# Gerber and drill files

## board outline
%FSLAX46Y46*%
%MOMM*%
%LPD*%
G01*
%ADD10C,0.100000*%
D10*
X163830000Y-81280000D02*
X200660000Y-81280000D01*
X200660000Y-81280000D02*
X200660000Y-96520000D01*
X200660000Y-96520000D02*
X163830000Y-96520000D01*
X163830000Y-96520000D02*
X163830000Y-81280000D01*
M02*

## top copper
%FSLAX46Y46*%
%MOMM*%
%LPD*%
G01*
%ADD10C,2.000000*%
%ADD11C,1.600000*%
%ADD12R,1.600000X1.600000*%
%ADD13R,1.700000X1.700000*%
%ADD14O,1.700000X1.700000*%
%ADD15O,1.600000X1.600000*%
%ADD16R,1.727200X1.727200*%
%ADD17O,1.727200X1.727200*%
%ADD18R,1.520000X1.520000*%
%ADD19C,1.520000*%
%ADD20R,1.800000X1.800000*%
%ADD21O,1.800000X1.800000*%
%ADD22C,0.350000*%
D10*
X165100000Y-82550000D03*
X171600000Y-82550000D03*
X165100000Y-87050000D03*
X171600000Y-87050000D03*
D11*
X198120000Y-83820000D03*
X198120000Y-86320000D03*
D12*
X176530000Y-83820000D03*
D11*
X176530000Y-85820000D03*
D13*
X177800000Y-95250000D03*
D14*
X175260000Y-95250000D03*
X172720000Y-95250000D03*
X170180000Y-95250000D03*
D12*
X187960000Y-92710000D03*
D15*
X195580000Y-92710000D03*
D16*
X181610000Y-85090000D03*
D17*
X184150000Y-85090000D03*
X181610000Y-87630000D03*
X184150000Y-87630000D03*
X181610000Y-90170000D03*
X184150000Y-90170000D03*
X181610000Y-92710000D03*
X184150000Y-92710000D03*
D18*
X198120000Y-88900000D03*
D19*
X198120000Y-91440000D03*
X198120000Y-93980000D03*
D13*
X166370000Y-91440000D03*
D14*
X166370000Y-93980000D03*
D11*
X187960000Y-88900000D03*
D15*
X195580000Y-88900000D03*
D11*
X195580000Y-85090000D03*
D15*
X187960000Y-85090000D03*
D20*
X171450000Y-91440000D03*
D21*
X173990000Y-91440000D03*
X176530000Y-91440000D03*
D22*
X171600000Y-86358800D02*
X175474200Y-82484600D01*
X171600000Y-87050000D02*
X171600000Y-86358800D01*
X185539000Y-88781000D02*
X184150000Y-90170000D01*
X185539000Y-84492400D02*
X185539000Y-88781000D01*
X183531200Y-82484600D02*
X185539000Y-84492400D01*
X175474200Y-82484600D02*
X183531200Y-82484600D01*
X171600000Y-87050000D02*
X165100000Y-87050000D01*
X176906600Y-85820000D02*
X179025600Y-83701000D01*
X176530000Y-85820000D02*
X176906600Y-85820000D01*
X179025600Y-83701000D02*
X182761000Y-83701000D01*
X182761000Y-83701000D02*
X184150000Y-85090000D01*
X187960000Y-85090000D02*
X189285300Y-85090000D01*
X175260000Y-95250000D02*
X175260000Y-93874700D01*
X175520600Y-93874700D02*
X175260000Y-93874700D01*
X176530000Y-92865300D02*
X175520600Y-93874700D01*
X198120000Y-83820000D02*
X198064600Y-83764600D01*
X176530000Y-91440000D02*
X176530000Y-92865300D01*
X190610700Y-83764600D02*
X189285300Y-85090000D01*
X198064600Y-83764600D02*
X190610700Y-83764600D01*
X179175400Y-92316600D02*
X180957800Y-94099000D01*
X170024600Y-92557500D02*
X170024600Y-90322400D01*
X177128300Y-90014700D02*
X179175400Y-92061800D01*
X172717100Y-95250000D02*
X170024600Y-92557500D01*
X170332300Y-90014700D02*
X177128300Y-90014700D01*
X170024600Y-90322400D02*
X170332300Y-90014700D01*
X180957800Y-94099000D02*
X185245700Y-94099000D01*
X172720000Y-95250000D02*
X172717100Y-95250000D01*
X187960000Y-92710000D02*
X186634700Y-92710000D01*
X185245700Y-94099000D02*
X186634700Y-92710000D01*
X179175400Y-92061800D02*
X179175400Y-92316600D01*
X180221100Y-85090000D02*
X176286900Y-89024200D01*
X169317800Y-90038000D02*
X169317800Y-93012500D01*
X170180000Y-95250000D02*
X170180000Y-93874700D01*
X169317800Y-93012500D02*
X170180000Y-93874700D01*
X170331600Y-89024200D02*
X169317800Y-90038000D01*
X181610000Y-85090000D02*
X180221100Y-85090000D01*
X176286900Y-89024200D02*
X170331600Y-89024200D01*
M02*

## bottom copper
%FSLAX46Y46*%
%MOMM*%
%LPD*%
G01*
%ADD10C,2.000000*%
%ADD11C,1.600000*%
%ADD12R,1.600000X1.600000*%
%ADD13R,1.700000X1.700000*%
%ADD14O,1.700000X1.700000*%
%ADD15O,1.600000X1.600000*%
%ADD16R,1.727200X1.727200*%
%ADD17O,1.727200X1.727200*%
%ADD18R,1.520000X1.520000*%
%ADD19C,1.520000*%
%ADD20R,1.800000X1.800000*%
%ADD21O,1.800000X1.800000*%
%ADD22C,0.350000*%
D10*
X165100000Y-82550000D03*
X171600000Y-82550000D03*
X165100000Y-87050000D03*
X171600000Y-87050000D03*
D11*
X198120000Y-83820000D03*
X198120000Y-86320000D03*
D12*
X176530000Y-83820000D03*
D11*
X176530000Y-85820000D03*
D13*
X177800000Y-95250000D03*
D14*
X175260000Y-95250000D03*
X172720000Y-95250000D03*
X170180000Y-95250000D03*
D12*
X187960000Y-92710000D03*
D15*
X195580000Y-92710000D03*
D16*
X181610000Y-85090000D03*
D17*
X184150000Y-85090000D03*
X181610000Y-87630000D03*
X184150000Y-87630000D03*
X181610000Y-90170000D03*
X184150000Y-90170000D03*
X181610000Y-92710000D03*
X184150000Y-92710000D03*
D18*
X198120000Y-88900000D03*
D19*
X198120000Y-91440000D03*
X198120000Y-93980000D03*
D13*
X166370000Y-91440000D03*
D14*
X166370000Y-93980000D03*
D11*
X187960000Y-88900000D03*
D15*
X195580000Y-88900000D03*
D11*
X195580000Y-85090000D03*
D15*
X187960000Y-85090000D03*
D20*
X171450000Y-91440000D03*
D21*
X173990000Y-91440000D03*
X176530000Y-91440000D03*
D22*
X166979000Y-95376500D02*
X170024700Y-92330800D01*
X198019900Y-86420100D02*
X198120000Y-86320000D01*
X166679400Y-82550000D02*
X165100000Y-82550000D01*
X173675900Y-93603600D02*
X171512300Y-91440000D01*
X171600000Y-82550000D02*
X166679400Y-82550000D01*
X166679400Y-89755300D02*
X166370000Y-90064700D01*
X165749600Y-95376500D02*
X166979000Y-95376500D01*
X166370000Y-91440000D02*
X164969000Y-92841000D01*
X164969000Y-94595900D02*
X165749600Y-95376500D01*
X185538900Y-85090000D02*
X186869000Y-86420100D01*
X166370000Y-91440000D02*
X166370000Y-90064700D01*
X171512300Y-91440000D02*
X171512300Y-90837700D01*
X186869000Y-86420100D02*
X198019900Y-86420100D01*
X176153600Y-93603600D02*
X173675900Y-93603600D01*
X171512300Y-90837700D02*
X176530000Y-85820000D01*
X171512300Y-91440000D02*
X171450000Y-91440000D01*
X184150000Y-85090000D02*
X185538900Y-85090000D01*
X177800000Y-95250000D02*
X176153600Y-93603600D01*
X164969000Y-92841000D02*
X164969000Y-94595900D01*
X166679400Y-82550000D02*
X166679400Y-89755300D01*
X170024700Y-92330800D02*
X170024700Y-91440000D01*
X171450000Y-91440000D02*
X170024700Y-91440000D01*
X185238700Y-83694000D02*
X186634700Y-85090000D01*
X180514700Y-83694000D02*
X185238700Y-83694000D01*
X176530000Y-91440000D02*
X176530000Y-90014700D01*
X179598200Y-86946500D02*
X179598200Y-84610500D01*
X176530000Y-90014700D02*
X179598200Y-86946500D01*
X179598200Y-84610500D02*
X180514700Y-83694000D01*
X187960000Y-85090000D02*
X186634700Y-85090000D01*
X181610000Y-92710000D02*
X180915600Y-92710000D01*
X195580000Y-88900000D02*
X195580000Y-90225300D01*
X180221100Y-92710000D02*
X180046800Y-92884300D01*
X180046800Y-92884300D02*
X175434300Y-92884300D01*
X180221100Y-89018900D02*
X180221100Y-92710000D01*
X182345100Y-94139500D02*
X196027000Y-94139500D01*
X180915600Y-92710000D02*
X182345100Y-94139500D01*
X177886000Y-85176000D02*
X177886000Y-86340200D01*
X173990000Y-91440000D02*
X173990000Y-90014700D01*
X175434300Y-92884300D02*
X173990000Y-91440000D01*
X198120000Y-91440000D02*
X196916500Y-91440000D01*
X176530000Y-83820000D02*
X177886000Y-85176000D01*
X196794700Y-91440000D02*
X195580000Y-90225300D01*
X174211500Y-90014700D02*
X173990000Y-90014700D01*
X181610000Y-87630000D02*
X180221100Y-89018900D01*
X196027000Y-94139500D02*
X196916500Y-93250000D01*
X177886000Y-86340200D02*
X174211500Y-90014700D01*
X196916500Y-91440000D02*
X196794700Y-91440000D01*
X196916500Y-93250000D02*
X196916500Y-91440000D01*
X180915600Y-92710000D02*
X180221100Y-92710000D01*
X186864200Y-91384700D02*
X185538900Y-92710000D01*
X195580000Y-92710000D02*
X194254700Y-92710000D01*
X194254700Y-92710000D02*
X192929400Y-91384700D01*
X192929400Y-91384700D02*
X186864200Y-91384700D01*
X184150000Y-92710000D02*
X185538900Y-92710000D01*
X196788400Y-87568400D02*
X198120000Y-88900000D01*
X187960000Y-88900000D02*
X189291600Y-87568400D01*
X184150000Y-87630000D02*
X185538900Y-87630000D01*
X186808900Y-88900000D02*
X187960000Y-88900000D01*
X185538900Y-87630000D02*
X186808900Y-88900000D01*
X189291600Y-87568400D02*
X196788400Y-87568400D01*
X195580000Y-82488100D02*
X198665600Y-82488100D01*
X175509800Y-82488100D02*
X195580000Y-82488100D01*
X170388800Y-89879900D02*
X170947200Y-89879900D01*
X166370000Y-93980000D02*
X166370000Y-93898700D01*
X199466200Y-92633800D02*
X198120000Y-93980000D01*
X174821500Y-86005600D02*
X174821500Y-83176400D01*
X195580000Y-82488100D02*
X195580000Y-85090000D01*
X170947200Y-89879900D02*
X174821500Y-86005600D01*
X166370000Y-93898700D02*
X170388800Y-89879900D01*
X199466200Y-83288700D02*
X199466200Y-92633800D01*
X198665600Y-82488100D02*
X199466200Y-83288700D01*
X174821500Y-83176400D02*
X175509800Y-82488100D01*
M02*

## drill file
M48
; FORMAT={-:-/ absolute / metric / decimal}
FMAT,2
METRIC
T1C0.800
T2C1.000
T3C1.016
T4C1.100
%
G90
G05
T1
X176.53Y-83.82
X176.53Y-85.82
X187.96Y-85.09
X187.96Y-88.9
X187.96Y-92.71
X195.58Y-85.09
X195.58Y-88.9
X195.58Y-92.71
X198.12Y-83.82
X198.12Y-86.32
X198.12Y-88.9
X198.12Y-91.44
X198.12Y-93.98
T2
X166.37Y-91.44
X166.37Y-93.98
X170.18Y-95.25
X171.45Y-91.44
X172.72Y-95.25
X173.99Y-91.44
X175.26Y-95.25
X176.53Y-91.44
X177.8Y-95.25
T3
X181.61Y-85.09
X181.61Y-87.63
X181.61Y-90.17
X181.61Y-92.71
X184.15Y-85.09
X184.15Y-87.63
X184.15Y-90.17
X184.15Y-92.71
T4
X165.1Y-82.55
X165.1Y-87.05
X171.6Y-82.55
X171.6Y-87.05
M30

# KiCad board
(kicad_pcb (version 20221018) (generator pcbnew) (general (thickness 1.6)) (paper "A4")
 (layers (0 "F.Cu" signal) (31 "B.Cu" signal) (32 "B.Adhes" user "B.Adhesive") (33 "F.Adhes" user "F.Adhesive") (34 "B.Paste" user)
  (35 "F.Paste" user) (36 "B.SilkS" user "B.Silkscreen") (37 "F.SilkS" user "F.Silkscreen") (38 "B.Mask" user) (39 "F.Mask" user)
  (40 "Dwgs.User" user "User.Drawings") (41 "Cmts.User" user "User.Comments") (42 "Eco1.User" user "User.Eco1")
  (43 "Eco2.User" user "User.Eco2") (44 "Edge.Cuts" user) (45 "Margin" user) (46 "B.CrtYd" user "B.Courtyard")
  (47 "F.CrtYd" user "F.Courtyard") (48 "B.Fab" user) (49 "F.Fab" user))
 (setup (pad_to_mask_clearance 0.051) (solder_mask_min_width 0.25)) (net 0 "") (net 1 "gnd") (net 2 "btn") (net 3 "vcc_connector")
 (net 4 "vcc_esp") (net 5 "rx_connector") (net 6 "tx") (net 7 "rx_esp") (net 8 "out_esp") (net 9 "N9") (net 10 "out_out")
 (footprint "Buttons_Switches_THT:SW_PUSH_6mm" (layer "F.Cu") (at 165.1 82.55)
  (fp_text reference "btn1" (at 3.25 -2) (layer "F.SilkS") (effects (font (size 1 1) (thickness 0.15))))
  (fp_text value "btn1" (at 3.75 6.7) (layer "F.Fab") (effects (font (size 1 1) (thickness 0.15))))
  (pad "1" thru_hole circle (at 0 0 90) (size 2 2) (drill 1.1) (layers "*.Cu" "*.Mask") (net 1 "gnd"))
  (pad "1" thru_hole circle (at 6.5 0 90) (size 2 2) (drill 1.1) (layers "*.Cu" "*.Mask") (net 1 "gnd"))
  (pad "2" thru_hole circle (at 0 4.5 90) (size 2 2) (drill 1.1) (layers "*.Cu" "*.Mask") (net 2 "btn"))
  (pad "2" thru_hole circle (at 6.5 4.5 90) (size 2 2) (drill 1.1) (layers "*.Cu" "*.Mask") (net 2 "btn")))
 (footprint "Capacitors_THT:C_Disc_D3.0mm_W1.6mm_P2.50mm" (layer "F.Cu") (at 198.12 83.82 -90)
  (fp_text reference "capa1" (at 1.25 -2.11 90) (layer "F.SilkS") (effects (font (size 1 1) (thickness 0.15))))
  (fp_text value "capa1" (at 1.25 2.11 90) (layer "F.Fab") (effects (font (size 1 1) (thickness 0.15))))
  (pad "1" thru_hole circle (at 0 0 270) (size 1.6 1.6) (drill 0.8) (layers "*.Cu" "*.Mask") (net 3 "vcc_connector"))
  (pad "2" thru_hole circle (at 2.5 0 270) (size 1.6 1.6) (drill 0.8) (layers "*.Cu" "*.Mask") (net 1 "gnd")))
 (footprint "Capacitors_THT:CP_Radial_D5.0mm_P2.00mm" (layer "F.Cu") (at 176.53 83.82 -90)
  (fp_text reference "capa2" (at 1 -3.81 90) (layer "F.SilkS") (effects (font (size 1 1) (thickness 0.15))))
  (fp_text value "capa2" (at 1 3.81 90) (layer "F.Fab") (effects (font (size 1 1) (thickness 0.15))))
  (pad "1" thru_hole rect (at 0 0 270) (size 1.6 1.6) (drill 0.8) (layers "*.Cu" "*.Mask") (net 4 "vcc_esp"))
  (pad "2" thru_hole circle (at 2 0 270) (size 1.6 1.6) (drill 0.8) (layers "*.Cu" "*.Mask") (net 1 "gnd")))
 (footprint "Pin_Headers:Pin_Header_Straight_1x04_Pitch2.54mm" (layer "F.Cu") (at 177.8 95.25 -90)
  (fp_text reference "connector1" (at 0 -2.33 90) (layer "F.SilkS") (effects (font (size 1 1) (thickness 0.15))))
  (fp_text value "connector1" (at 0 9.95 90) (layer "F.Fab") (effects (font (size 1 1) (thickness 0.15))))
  (pad "1" thru_hole rect (at 0 0 270) (size 1.7 1.7) (drill 1) (layers "*.Cu" "*.Mask") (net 1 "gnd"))
  (pad "2" thru_hole oval (at 0 2.54 270) (size 1.7 1.7) (drill 1) (layers "*.Cu" "*.Mask") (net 3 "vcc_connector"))
  (pad "3" thru_hole oval (at 0 5.08 270) (size 1.7 1.7) (drill 1) (layers "*.Cu" "*.Mask") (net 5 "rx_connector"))
  (pad "4" thru_hole oval (at 0 7.62 270) (size 1.7 1.7) (drill 1) (layers "*.Cu" "*.Mask") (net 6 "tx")))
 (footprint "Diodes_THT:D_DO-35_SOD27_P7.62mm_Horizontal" (layer "F.Cu") (at 187.96 92.71)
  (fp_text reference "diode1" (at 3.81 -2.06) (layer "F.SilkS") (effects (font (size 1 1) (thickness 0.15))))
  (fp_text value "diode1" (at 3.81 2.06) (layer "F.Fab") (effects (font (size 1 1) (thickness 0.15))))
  (pad "1" thru_hole rect (at 0 0) (size 1.6 1.6) (drill 0.8) (layers "*.Cu" "*.Mask") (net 5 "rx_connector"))
  (pad "2" thru_hole oval (at 7.62 0) (size 1.6 1.6) (drill 0.8) (layers "*.Cu" "*.Mask") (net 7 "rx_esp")))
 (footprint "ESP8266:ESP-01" (layer "F.Cu") (at 181.61 85.09)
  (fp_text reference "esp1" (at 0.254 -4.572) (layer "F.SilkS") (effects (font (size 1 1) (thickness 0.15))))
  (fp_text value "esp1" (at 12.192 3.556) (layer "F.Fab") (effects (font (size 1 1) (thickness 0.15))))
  (pad "1" thru_hole rect (at 0 0) (size 1.7272 1.7272) (drill 1.016) (layers "*.Cu" "*.Mask" "F.SilkS") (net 6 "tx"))
  (pad "2" thru_hole oval (at 2.54 0) (size 1.7272 1.7272) (drill 1.016) (layers "*.Cu" "*.Mask" "F.SilkS") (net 1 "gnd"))
  (pad "3" thru_hole oval (at 0 2.54) (size 1.7272 1.7272) (drill 1.016) (layers "*.Cu" "*.Mask" "F.SilkS") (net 4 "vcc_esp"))
  (pad "4" thru_hole oval (at 2.54 2.54) (size 1.7272 1.7272) (drill 1.016) (layers "*.Cu" "*.Mask" "F.SilkS") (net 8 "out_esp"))
  (pad "5" thru_hole oval (at 0 5.08) (size 1.7272 1.7272) (drill 1.016) (layers "*.Cu" "*.Mask" "F.SilkS") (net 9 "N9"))
  (pad "6" thru_hole oval (at 2.54 5.08) (size 1.7272 1.7272) (drill 1.016) (layers "*.Cu" "*.Mask" "F.SilkS") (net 2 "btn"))
  (pad "7" thru_hole oval (at 0 7.62) (size 1.7272 1.7272) (drill 1.016) (layers "*.Cu" "*.Mask" "F.SilkS") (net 4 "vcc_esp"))
  (pad "8" thru_hole oval (at 2.54 7.62) (size 1.7272 1.7272) (drill 1.016) (layers "*.Cu" "*.Mask" "F.SilkS") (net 7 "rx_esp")))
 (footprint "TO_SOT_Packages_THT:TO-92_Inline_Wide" (layer "F.Cu") (at 198.12 88.9 -90)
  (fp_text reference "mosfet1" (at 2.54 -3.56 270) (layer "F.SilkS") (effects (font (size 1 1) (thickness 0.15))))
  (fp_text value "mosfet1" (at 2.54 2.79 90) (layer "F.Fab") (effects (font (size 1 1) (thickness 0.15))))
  (pad "1" thru_hole rect (at 0 0) (size 1.52 1.52) (drill 0.8) (layers "*.Cu" "*.Mask") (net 8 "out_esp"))
  (pad "2" thru_hole circle (at 2.54 0) (size 1.52 1.52) (drill 0.8) (layers "*.Cu" "*.Mask") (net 4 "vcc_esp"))
  (pad "3" thru_hole circle (at 5.08 0) (size 1.52 1.52) (drill 0.8) (layers "*.Cu" "*.Mask") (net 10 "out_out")))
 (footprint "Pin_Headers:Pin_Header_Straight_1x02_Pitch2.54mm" (layer "F.Cu") (at 166.37 91.44)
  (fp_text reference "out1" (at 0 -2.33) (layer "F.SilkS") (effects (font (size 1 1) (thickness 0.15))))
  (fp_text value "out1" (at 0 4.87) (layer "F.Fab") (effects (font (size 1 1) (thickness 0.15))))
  (pad "1" thru_hole rect (at 0 0) (size 1.7 1.7) (drill 1) (layers "*.Cu" "*.Mask") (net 1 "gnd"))
  (pad "2" thru_hole oval (at 0 2.54) (size 1.7 1.7) (drill 1) (layers "*.Cu" "*.Mask") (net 10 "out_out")))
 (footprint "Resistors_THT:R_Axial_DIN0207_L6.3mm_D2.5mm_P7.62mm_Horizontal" (layer "F.Cu") (at 187.96 88.9)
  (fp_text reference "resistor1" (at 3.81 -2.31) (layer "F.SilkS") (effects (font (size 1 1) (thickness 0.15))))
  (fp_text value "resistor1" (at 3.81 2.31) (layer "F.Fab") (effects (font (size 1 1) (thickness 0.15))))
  (pad "1" thru_hole circle (at 0 0) (size 1.6 1.6) (drill 0.8) (layers "*.Cu" "*.Mask") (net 8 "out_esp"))
  (pad "2" thru_hole oval (at 7.62 0) (size 1.6 1.6) (drill 0.8) (layers "*.Cu" "*.Mask") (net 4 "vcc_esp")))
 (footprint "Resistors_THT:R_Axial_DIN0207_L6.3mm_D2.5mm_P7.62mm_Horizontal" (layer "F.Cu") (at 195.58 85.09 180)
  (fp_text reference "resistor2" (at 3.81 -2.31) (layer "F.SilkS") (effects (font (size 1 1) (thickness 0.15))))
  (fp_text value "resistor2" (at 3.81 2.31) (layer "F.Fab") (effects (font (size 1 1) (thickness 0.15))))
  (pad "1" thru_hole circle (at 0 0 180) (size 1.6 1.6) (drill 0.8) (layers "*.Cu" "*.Mask") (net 10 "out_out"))
  (pad "2" thru_hole oval (at 7.62 0 180) (size 1.6 1.6) (drill 0.8) (layers "*.Cu" "*.Mask") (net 3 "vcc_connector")))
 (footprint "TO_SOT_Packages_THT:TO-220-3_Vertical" (layer "F.Cu") (at 171.45 91.44)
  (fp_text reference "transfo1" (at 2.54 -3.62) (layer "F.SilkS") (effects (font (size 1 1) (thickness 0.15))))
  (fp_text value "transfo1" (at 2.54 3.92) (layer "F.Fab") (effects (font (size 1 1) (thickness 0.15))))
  (pad "1" thru_hole rect (at 0 0) (size 1.8 1.8) (drill 1) (layers "*.Cu" "*.Mask") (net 1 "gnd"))
  (pad "2" thru_hole oval (at 2.54 0) (size 1.8 1.8) (drill 1) (layers "*.Cu" "*.Mask") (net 4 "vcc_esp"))
  (pad "3" thru_hole oval (at 5.08 0) (size 1.8 1.8) (drill 1) (layers "*.Cu" "*.Mask") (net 3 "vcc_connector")))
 (gr_line (start 163.83 81.28) (end 200.66 81.28) (stroke (width 0.1) (type solid)) (layer "Edge.Cuts"))
 (gr_line (start 200.66 81.28) (end 200.66 96.52) (stroke (width 0.1) (type solid)) (layer "Edge.Cuts"))
 (gr_line (start 200.66 96.52) (end 163.83 96.52) (stroke (width 0.1) (type solid)) (layer "Edge.Cuts"))
 (gr_line (start 163.83 96.52) (end 163.83 81.28) (stroke (width 0.1) (type solid)) (layer "Edge.Cuts"))
 (segment (start 171.6 86.3588) (end 175.4742 82.4846) (width 0.35) (layer "F.Cu") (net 2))
 (segment (start 171.6 87.05) (end 171.6 86.3588) (width 0.35) (layer "F.Cu") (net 2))
 (segment (start 185.539 88.781) (end 184.15 90.17) (width 0.35) (layer "F.Cu") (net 2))
 (segment (start 185.539 84.4924) (end 185.539 88.781) (width 0.35) (layer "F.Cu") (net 2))
 (segment (start 183.5312 82.4846) (end 185.539 84.4924) (width 0.35) (layer "F.Cu") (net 2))
 (segment (start 175.4742 82.4846) (end 183.5312 82.4846) (width 0.35) (layer "F.Cu") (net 2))
 (segment (start 171.6 87.05) (end 165.1 87.05) (width 0.35) (layer "F.Cu") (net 2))
 (segment (start 176.9066 85.82) (end 179.0256 83.701) (width 0.35) (layer "F.Cu") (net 1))
 (segment (start 176.53 85.82) (end 176.9066 85.82) (width 0.35) (layer "F.Cu") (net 1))
 (segment (start 179.0256 83.701) (end 182.761 83.701) (width 0.35) (layer "F.Cu") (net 1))
 (segment (start 182.761 83.701) (end 184.15 85.09) (width 0.35) (layer "F.Cu") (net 1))
 (segment (start 166.979 95.3765) (end 170.0247 92.3308) (width 0.35) (layer "B.Cu") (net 1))
 (segment (start 198.0199 86.4201) (end 198.12 86.32) (width 0.35) (layer "B.Cu") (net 1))
 (segment (start 166.6794 82.55) (end 165.1 82.55) (width 0.35) (layer "B.Cu") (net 1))
 (segment (start 173.6759 93.6036) (end 171.5123 91.44) (width 0.35) (layer "B.Cu") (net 1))
 (segment (start 171.6 82.55) (end 166.6794 82.55) (width 0.35) (layer "B.Cu") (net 1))
 (segment (start 166.6794 89.7553) (end 166.37 90.0647) (width 0.35) (layer "B.Cu") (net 1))
 (segment (start 165.7496 95.3765) (end 166.979 95.3765) (width 0.35) (layer "B.Cu") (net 1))
 (segment (start 166.37 91.44) (end 164.969 92.841) (width 0.35) (layer "B.Cu") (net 1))
 (segment (start 164.969 94.5959) (end 165.7496 95.3765) (width 0.35) (layer "B.Cu") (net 1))
 (segment (start 185.5389 85.09) (end 186.869 86.4201) (width 0.35) (layer "B.Cu") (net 1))
 (segment (start 166.37 91.44) (end 166.37 90.0647) (width 0.35) (layer "B.Cu") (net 1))
 (segment (start 171.5123 91.44) (end 171.5123 90.8377) (width 0.35) (layer "B.Cu") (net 1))
 (segment (start 186.869 86.4201) (end 198.0199 86.4201) (width 0.35) (layer "B.Cu") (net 1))
 (segment (start 176.1536 93.6036) (end 173.6759 93.6036) (width 0.35) (layer "B.Cu") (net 1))
 (segment (start 171.5123 90.8377) (end 176.53 85.82) (width 0.35) (layer "B.Cu") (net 1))
 (segment (start 171.5123 91.44) (end 171.45 91.44) (width 0.35) (layer "B.Cu") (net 1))
 (segment (start 184.15 85.09) (end 185.5389 85.09) (width 0.35) (layer "B.Cu") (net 1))
 (segment (start 177.8 95.25) (end 176.1536 93.6036) (width 0.35) (layer "B.Cu") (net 1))
 (segment (start 164.969 92.841) (end 164.969 94.5959) (width 0.35) (layer "B.Cu") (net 1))
 (segment (start 166.6794 82.55) (end 166.6794 89.7553) (width 0.35) (layer "B.Cu") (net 1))
 (segment (start 170.0247 92.3308) (end 170.0247 91.44) (width 0.35) (layer "B.Cu") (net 1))
 (segment (start 171.45 91.44) (end 170.0247 91.44) (width 0.35) (layer "B.Cu") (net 1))
 (segment (start 187.96 85.09) (end 189.2853 85.09) (width 0.35) (layer "F.Cu") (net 3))
 (segment (start 175.26 95.25) (end 175.26 93.8747) (width 0.35) (layer "F.Cu") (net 3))
 (segment (start 175.5206 93.8747) (end 175.26 93.8747) (width 0.35) (layer "F.Cu") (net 3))
 (segment (start 176.53 92.8653) (end 175.5206 93.8747) (width 0.35) (layer "F.Cu") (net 3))
 (segment (start 198.12 83.82) (end 198.0646 83.7646) (width 0.35) (layer "F.Cu") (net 3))
 (segment (start 176.53 91.44) (end 176.53 92.8653) (width 0.35) (layer "F.Cu") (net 3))
 (segment (start 190.6107 83.7646) (end 189.2853 85.09) (width 0.35) (layer "F.Cu") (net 3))
 (segment (start 198.0646 83.7646) (end 190.6107 83.7646) (width 0.35) (layer "F.Cu") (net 3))
 (segment (start 185.2387 83.694) (end 186.6347 85.09) (width 0.35) (layer "B.Cu") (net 3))
 (segment (start 180.5147 83.694) (end 185.2387 83.694) (width 0.35) (layer "B.Cu") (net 3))
 (segment (start 176.53 91.44) (end 176.53 90.0147) (width 0.35) (layer "B.Cu") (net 3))
 (segment (start 179.5982 86.9465) (end 179.5982 84.6105) (width 0.35) (layer "B.Cu") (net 3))
 (segment (start 176.53 90.0147) (end 179.5982 86.9465) (width 0.35) (layer "B.Cu") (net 3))
 (segment (start 179.5982 84.6105) (end 180.5147 83.694) (width 0.35) (layer "B.Cu") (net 3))
 (segment (start 187.96 85.09) (end 186.6347 85.09) (width 0.35) (layer "B.Cu") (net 3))
 (segment (start 181.61 92.71) (end 180.9156 92.71) (width 0.35) (layer "B.Cu") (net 4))
 (segment (start 195.58 88.9) (end 195.58 90.2253) (width 0.35) (layer "B.Cu") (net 4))
 (segment (start 180.2211 92.71) (end 180.0468 92.8843) (width 0.35) (layer "B.Cu") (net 4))
 (segment (start 180.0468 92.8843) (end 175.4343 92.8843) (width 0.35) (layer "B.Cu") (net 4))
 (segment (start 180.2211 89.0189) (end 180.2211 92.71) (width 0.35) (layer "B.Cu") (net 4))
 (segment (start 182.3451 94.1395) (end 196.027 94.1395) (width 0.35) (layer "B.Cu") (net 4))
 (segment (start 180.9156 92.71) (end 182.3451 94.1395) (width 0.35) (layer "B.Cu") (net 4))
 (segment (start 177.886 85.176) (end 177.886 86.3402) (width 0.35) (layer "B.Cu") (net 4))
 (segment (start 173.99 91.44) (end 173.99 90.0147) (width 0.35) (layer "B.Cu") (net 4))
 (segment (start 175.4343 92.8843) (end 173.99 91.44) (width 0.35) (layer "B.Cu") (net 4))
 (segment (start 198.12 91.44) (end 196.9165 91.44) (width 0.35) (layer "B.Cu") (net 4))
 (segment (start 176.53 83.82) (end 177.886 85.176) (width 0.35) (layer "B.Cu") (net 4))
 (segment (start 196.7947 91.44) (end 195.58 90.2253) (width 0.35) (layer "B.Cu") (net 4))
 (segment (start 174.2115 90.0147) (end 173.99 90.0147) (width 0.35) (layer "B.Cu") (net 4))
 (segment (start 181.61 87.63) (end 180.2211 89.0189) (width 0.35) (layer "B.Cu") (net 4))
 (segment (start 196.027 94.1395) (end 196.9165 93.25) (width 0.35) (layer "B.Cu") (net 4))
 (segment (start 177.886 86.3402) (end 174.2115 90.0147) (width 0.35) (layer "B.Cu") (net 4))
 (segment (start 196.9165 91.44) (end 196.7947 91.44) (width 0.35) (layer "B.Cu") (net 4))
 (segment (start 196.9165 93.25) (end 196.9165 91.44) (width 0.35) (layer "B.Cu") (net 4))
 (segment (start 180.9156 92.71) (end 180.2211 92.71) (width 0.35) (layer "B.Cu") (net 4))
 (segment (start 179.1754 92.3166) (end 180.9578 94.099) (width 0.35) (layer "F.Cu") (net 5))
 (segment (start 170.0246 92.5575) (end 170.0246 90.3224) (width 0.35) (layer "F.Cu") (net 5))
 (segment (start 177.1283 90.0147) (end 179.1754 92.0618) (width 0.35) (layer "F.Cu") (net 5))
 (segment (start 172.7171 95.25) (end 170.0246 92.5575) (width 0.35) (layer "F.Cu") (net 5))
 (segment (start 170.3323 90.0147) (end 177.1283 90.0147) (width 0.35) (layer "F.Cu") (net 5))
 (segment (start 170.0246 90.3224) (end 170.3323 90.0147) (width 0.35) (layer "F.Cu") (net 5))
 (segment (start 180.9578 94.099) (end 185.2457 94.099) (width 0.35) (layer "F.Cu") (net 5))
 (segment (start 172.72 95.25) (end 172.7171 95.25) (width 0.35) (layer "F.Cu") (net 5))
 (segment (start 187.96 92.71) (end 186.6347 92.71) (width 0.35) (layer "F.Cu") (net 5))
 (segment (start 185.2457 94.099) (end 186.6347 92.71) (width 0.35) (layer "F.Cu") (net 5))
 (segment (start 179.1754 92.0618) (end 179.1754 92.3166) (width 0.35) (layer "F.Cu") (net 5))
 (segment (start 180.2211 85.09) (end 176.2869 89.0242) (width 0.35) (layer "F.Cu") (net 6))
 (segment (start 169.3178 90.038) (end 169.3178 93.0125) (width 0.35) (layer "F.Cu") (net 6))
 (segment (start 170.18 95.25) (end 170.18 93.8747) (width 0.35) (layer "F.Cu") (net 6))
 (segment (start 169.3178 93.0125) (end 170.18 93.8747) (width 0.35) (layer "F.Cu") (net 6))
 (segment (start 170.3316 89.0242) (end 169.3178 90.038) (width 0.35) (layer "F.Cu") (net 6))
 (segment (start 181.61 85.09) (end 180.2211 85.09) (width 0.35) (layer "F.Cu") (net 6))
 (segment (start 176.2869 89.0242) (end 170.3316 89.0242) (width 0.35) (layer "F.Cu") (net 6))
 (segment (start 186.8642 91.3847) (end 185.5389 92.71) (width 0.35) (layer "B.Cu") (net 7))
 (segment (start 195.58 92.71) (end 194.2547 92.71) (width 0.35) (layer "B.Cu") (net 7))
 (segment (start 194.2547 92.71) (end 192.9294 91.3847) (width 0.35) (layer "B.Cu") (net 7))
 (segment (start 192.9294 91.3847) (end 186.8642 91.3847) (width 0.35) (layer "B.Cu") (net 7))
 (segment (start 184.15 92.71) (end 185.5389 92.71) (width 0.35) (layer "B.Cu") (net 7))
 (segment (start 196.7884 87.5684) (end 198.12 88.9) (width 0.35) (layer "B.Cu") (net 8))
 (segment (start 187.96 88.9) (end 189.2916 87.5684) (width 0.35) (layer "B.Cu") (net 8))
 (segment (start 184.15 87.63) (end 185.5389 87.63) (width 0.35) (layer "B.Cu") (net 8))
 (segment (start 186.8089 88.9) (end 187.96 88.9) (width 0.35) (layer "B.Cu") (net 8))
 (segment (start 185.5389 87.63) (end 186.8089 88.9) (width 0.35) (layer "B.Cu") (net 8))
 (segment (start 189.2916 87.5684) (end 196.7884 87.5684) (width 0.35) (layer "B.Cu") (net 8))
 (segment (start 195.58 82.4881) (end 198.6656 82.4881) (width 0.35) (layer "B.Cu") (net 10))
 (segment (start 175.5098 82.4881) (end 195.58 82.4881) (width 0.35) (layer "B.Cu") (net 10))
 (segment (start 170.3888 89.8799) (end 170.9472 89.8799) (width 0.35) (layer "B.Cu") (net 10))
 (segment (start 166.37 93.98) (end 166.37 93.8987) (width 0.35) (layer "B.Cu") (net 10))
 (segment (start 199.4662 92.6338) (end 198.12 93.98) (width 0.35) (layer "B.Cu") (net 10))
 (segment (start 174.8215 86.0056) (end 174.8215 83.1764) (width 0.35) (layer "B.Cu") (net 10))
 (segment (start 195.58 82.4881) (end 195.58 85.09) (width 0.35) (layer "B.Cu") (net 10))
 (segment (start 170.9472 89.8799) (end 174.8215 86.0056) (width 0.35) (layer "B.Cu") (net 10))
 (segment (start 166.37 93.8987) (end 170.3888 89.8799) (width 0.35) (layer "B.Cu") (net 10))
 (segment (start 199.4662 83.2887) (end 199.4662 92.6338) (width 0.35) (layer "B.Cu") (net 10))
 (segment (start 198.6656 82.4881) (end 199.4662 83.2887) (width 0.35) (layer "B.Cu") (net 10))
 (segment (start 174.8215 83.1764) (end 175.5098 82.4881) (width 0.35) (layer "B.Cu") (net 10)))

